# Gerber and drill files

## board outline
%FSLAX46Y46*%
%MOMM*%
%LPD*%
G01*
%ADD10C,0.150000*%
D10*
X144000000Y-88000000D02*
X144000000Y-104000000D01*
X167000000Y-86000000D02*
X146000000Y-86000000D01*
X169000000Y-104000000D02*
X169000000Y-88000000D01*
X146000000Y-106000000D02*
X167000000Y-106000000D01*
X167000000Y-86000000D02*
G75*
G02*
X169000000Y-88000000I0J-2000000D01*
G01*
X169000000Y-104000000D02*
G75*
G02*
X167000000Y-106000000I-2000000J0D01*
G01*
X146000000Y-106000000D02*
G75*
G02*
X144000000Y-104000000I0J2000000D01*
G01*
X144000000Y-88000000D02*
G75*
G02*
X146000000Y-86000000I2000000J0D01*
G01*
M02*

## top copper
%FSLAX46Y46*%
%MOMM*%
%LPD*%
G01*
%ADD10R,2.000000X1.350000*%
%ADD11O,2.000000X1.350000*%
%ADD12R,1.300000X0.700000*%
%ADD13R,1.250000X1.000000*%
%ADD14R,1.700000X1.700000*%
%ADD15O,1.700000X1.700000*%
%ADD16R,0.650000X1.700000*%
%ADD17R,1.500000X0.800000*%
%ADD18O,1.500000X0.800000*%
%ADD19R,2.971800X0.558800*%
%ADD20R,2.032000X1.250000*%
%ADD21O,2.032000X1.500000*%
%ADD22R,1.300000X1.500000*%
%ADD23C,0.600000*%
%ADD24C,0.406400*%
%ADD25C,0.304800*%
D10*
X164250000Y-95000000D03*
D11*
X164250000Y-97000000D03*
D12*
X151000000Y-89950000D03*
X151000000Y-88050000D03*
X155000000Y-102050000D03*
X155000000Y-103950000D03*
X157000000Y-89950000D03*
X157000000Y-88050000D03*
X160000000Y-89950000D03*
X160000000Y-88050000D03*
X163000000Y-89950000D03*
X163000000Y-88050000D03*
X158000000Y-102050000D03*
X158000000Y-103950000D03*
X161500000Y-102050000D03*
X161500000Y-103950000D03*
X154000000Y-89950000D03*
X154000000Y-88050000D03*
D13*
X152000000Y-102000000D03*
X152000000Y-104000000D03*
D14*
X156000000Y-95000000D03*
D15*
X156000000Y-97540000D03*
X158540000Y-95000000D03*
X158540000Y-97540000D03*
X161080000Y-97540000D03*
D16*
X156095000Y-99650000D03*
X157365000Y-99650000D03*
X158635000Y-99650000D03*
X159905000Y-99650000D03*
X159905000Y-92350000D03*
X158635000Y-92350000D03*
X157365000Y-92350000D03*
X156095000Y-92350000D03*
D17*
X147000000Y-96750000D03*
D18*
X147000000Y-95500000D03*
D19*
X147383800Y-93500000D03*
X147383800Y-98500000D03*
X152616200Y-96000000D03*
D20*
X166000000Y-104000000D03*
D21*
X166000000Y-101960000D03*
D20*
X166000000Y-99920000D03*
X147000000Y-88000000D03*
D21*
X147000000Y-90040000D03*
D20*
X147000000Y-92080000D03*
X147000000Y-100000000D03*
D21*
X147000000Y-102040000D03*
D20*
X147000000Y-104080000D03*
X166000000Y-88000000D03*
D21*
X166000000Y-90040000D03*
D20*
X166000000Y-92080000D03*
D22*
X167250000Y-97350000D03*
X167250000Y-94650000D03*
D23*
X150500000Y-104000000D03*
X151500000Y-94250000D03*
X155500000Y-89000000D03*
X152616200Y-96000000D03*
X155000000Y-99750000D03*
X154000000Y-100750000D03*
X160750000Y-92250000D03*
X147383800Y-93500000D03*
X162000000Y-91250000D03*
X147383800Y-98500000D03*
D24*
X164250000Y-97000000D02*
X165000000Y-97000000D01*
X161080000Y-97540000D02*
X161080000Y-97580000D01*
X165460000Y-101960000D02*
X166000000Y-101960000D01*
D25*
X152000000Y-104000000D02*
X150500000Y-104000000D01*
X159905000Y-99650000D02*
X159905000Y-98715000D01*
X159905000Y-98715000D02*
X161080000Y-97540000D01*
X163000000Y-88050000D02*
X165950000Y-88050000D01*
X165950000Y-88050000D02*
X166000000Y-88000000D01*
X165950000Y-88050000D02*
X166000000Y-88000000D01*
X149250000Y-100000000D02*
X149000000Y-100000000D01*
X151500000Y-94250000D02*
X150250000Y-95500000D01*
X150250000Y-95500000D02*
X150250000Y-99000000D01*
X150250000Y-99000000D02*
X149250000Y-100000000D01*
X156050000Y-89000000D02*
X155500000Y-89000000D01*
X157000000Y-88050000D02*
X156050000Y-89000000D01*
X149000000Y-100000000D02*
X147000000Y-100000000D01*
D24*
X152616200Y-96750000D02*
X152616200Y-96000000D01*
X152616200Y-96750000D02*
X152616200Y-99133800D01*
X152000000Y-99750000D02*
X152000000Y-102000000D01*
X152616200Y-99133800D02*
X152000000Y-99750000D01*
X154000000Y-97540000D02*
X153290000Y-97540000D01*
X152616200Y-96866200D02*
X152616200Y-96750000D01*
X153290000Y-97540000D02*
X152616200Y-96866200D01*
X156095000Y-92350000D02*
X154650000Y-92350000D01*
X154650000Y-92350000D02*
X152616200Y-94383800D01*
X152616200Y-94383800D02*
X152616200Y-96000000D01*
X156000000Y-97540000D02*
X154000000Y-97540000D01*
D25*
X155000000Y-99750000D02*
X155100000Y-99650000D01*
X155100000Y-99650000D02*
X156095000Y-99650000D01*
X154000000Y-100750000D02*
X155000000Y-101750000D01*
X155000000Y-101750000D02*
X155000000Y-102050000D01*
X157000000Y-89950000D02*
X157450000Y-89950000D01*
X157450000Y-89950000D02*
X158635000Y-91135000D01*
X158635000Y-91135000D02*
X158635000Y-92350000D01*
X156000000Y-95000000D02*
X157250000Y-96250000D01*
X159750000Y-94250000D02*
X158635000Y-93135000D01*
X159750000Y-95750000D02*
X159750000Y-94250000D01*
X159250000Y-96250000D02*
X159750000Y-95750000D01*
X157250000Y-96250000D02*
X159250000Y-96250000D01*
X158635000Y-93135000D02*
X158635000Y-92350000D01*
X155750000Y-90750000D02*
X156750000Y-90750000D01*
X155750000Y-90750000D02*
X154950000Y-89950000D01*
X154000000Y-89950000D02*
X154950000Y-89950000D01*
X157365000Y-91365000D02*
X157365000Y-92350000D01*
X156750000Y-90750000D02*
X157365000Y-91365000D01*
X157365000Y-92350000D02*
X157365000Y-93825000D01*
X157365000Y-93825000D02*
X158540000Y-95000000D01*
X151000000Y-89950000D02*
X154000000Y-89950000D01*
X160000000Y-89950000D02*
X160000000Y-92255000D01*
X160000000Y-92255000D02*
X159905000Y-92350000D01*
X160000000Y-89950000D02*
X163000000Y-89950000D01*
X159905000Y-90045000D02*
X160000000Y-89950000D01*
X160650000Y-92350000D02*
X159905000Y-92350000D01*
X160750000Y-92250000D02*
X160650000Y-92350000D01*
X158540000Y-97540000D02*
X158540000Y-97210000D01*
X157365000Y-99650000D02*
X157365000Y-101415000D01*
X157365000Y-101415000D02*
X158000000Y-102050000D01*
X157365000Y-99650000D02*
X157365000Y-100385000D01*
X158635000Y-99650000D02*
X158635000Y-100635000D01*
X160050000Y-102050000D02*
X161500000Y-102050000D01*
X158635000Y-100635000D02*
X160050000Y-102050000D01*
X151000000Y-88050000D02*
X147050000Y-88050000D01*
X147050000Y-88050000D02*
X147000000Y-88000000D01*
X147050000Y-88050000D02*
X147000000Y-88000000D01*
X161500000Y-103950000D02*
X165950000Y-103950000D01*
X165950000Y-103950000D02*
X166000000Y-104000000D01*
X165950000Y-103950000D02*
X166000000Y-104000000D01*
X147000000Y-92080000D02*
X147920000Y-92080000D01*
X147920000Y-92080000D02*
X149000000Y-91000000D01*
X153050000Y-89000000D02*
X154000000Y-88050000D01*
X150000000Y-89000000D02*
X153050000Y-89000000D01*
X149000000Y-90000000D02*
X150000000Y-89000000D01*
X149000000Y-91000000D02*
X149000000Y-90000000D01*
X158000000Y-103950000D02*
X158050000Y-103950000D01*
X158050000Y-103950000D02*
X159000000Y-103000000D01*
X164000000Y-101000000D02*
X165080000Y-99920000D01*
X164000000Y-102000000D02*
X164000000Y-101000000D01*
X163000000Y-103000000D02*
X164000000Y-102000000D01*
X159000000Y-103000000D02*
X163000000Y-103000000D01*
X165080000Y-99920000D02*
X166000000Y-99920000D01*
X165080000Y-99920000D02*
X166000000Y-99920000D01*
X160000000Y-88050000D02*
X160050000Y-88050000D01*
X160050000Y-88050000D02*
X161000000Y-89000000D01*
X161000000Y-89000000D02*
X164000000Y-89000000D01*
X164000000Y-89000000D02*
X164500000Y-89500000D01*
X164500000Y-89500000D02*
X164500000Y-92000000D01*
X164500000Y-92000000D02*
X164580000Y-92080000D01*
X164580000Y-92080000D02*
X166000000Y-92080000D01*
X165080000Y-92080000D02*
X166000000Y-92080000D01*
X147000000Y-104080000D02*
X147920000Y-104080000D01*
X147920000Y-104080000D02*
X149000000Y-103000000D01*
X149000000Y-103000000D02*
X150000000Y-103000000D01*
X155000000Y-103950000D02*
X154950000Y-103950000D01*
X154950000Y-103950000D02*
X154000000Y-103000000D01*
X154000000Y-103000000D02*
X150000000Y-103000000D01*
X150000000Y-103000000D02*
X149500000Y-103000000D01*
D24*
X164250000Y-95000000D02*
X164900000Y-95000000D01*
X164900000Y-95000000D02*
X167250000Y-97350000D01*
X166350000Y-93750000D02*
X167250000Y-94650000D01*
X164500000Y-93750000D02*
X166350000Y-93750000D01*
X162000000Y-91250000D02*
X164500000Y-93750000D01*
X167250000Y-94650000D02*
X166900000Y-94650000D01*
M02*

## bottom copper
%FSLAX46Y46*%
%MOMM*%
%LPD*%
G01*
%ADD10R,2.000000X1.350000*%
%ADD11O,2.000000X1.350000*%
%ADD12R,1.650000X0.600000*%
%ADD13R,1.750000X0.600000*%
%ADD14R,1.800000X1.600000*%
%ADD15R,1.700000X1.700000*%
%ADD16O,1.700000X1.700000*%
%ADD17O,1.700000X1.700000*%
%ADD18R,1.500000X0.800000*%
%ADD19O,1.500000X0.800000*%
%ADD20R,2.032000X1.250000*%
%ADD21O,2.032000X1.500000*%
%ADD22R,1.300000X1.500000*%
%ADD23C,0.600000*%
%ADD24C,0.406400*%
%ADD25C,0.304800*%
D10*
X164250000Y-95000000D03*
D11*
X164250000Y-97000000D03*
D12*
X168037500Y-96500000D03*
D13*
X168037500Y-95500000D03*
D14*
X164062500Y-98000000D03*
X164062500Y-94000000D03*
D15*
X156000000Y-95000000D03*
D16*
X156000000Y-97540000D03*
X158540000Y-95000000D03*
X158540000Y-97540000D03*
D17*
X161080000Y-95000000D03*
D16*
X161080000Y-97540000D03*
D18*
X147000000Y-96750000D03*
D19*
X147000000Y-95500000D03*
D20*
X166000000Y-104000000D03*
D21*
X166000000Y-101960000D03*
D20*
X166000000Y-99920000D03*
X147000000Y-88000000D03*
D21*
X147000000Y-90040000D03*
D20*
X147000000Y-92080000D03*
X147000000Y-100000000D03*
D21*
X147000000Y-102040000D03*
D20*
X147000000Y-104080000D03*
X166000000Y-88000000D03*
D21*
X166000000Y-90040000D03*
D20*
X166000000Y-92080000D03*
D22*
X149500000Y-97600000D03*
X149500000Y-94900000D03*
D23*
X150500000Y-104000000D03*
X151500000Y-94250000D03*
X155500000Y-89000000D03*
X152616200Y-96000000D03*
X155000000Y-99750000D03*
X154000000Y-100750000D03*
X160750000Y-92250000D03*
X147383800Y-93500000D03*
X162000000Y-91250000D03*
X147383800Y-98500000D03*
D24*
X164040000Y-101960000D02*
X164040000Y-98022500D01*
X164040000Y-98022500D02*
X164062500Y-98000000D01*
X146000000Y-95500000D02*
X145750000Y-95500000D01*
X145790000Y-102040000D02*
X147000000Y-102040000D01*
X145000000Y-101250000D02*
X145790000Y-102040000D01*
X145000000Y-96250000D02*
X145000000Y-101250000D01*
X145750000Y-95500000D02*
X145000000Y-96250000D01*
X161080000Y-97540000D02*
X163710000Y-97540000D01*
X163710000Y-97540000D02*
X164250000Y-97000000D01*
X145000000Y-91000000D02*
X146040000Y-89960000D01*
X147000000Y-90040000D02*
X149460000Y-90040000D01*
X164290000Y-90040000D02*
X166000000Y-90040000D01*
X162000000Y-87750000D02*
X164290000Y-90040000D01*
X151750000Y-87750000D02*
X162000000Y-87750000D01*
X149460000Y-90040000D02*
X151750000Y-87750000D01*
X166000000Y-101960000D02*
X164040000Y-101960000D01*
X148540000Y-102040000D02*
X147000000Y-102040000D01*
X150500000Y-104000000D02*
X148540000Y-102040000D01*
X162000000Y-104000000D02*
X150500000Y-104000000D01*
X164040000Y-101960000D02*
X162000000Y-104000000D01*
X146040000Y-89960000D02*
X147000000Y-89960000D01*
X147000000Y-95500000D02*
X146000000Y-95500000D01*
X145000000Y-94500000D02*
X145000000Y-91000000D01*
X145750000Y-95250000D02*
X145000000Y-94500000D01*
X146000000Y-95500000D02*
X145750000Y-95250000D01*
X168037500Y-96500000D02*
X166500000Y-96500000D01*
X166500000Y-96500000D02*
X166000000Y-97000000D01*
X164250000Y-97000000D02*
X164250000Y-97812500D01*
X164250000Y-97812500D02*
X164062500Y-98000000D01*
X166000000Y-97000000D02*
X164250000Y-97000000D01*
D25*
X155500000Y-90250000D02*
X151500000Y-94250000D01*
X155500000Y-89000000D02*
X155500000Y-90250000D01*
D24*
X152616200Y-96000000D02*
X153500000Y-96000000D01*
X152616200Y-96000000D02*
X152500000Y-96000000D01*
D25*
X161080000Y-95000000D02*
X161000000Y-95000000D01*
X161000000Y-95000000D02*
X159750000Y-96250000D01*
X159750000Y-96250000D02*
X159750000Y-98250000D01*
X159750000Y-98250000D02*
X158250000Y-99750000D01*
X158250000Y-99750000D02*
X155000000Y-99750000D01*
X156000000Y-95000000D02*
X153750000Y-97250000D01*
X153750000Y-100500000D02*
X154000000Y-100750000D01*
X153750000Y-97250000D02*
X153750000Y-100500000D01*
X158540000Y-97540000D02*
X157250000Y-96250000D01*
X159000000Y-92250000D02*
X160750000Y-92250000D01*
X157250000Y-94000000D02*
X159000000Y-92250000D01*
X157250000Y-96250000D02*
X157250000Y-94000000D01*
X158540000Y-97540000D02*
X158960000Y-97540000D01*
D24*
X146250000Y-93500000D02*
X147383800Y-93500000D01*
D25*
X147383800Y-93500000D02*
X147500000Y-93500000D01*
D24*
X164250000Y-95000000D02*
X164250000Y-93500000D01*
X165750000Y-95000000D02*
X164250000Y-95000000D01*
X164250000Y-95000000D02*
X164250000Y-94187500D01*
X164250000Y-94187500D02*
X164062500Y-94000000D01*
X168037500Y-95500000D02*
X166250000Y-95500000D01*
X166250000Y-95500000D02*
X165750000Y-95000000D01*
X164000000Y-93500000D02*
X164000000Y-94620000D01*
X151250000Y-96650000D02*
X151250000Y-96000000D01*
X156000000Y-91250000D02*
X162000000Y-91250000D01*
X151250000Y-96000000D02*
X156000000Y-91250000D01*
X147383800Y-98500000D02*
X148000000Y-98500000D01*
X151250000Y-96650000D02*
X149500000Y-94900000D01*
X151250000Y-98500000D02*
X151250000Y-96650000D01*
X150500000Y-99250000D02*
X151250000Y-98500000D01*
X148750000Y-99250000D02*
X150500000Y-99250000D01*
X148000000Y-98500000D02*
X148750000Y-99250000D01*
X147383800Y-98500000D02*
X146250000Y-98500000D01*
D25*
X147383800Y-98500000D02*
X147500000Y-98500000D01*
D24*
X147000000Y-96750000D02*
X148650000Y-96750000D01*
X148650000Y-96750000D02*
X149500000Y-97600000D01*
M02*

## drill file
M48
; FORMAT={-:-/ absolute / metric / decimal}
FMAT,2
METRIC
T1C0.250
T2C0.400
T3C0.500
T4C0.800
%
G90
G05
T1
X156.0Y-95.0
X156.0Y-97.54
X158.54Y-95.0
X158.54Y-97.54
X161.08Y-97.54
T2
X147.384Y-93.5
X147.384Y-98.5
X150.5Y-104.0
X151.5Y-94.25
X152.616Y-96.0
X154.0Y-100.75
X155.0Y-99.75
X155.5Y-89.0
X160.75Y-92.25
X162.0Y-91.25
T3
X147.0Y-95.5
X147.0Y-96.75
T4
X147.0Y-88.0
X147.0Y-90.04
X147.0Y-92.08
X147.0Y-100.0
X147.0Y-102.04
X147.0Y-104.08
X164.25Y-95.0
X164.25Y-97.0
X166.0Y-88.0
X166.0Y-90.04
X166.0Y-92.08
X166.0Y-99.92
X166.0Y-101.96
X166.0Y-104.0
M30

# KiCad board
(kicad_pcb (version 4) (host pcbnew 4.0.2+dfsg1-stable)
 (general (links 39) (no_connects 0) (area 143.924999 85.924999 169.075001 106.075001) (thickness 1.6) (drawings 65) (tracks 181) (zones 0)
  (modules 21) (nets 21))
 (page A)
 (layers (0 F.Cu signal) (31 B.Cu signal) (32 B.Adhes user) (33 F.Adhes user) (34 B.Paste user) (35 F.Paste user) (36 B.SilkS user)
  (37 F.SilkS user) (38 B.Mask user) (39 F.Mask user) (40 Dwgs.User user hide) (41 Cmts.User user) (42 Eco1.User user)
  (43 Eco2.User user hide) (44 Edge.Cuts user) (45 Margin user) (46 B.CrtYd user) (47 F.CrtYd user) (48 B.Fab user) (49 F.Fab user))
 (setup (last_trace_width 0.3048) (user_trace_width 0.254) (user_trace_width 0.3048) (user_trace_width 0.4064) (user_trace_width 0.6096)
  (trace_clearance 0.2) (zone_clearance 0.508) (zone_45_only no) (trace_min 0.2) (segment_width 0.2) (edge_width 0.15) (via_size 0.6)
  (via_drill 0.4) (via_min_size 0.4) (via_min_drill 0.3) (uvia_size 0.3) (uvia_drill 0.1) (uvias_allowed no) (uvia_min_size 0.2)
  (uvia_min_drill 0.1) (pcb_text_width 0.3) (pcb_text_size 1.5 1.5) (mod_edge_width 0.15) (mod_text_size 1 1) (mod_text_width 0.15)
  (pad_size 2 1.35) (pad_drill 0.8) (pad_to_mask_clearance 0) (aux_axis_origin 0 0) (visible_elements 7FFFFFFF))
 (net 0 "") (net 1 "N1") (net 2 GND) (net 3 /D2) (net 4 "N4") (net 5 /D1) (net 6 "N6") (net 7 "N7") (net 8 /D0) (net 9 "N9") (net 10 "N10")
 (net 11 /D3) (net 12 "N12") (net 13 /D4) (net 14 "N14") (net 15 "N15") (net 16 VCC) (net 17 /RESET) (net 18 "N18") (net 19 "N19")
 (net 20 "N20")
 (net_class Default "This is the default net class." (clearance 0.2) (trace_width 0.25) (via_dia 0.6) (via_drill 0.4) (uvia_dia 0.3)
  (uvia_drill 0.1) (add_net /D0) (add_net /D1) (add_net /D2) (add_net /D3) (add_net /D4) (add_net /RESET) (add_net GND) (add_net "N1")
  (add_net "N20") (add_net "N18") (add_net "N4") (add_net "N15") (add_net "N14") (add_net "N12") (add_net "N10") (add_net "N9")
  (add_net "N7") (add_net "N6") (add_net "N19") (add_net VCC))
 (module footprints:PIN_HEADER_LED (layer B.Cu) (at 164.25 95 180)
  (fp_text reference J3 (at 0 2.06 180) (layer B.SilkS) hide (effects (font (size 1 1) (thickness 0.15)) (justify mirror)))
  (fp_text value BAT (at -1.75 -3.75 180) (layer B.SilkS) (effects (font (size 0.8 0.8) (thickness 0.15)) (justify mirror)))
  (pad 1 thru_hole rect (at 0 0 180) (size 2 1.35) (drill 0.8) (layers *.Cu *.Mask) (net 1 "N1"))
  (pad 2 thru_hole oval (at 0 -2 180) (size 2 1.35) (drill 0.8) (layers *.Cu *.Mask) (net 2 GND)))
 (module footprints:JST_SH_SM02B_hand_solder (layer B.Cu) (at 166 96 90)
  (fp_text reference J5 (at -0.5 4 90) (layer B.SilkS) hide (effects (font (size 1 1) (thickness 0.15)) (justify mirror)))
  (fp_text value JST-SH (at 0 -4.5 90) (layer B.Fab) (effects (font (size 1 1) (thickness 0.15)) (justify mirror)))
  (pad 1 smd rect (at -0.5 2.0375 90) (size 0.6 1.65) (layers B.Cu B.Paste B.Mask) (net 2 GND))
  (pad 2 smd rect (at 0.5 2.0375 90) (size 0.6 1.75) (layers B.Cu B.Paste B.Mask) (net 1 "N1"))
  (pad 1 smd rect (at -2 -1.9375 90) (size 1.6 1.8) (layers B.Cu B.Paste B.Mask) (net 2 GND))
  (pad 2 smd rect (at 2 -1.9375 90) (size 1.6 1.8) (layers B.Cu B.Paste B.Mask) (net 1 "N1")))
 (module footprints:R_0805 (layer F.Cu) (at 151 89 90)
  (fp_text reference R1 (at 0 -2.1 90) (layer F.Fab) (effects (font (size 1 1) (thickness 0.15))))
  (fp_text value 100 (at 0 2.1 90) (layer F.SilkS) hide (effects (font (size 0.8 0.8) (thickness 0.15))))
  (pad 1 smd rect (at -0.95 0 90) (size 0.7 1.3) (layers F.Cu F.Paste F.Mask) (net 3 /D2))
  (pad 2 smd rect (at 0.95 0 90) (size 0.7 1.3) (layers F.Cu F.Paste F.Mask) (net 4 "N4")))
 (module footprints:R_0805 (layer F.Cu) (at 155 103 270)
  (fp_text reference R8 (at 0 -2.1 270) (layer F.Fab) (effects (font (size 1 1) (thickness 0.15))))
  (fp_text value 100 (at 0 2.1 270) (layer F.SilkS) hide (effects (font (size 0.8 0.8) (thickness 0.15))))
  (pad 1 smd rect (at -0.95 0 270) (size 0.7 1.3) (layers F.Cu F.Paste F.Mask) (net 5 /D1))
  (pad 2 smd rect (at 0.95 0 270) (size 0.7 1.3) (layers F.Cu F.Paste F.Mask) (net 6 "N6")))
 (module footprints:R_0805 (layer F.Cu) (at 157 89 90)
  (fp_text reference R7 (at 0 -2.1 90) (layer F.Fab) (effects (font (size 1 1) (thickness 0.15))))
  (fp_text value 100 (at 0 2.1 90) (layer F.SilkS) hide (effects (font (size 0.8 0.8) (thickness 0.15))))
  (pad 1 smd rect (at -0.95 0 90) (size 0.7 1.3) (layers F.Cu F.Paste F.Mask) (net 5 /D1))
  (pad 2 smd rect (at 0.95 0 90) (size 0.7 1.3) (layers F.Cu F.Paste F.Mask) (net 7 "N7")))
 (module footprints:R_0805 (layer F.Cu) (at 160 89 90)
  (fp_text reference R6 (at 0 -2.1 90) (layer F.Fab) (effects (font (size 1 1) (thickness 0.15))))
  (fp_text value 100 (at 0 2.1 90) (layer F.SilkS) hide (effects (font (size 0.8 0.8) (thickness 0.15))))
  (pad 1 smd rect (at -0.95 0 90) (size 0.7 1.3) (layers F.Cu F.Paste F.Mask) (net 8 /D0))
  (pad 2 smd rect (at 0.95 0 90) (size 0.7 1.3) (layers F.Cu F.Paste F.Mask) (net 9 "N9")))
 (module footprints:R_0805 (layer F.Cu) (at 163 89 90)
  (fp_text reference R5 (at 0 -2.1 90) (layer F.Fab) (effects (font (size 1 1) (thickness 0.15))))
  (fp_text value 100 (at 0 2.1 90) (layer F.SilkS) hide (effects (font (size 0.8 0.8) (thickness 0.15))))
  (pad 1 smd rect (at -0.95 0 90) (size 0.7 1.3) (layers F.Cu F.Paste F.Mask) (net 8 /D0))
  (pad 2 smd rect (at 0.95 0 90) (size 0.7 1.3) (layers F.Cu F.Paste F.Mask) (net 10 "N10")))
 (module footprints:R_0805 (layer F.Cu) (at 158 103 270)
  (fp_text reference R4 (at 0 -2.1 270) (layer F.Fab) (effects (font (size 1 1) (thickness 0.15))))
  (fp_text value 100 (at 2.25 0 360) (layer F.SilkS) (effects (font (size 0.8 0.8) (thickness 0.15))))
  (pad 1 smd rect (at -0.95 0 270) (size 0.7 1.3) (layers F.Cu F.Paste F.Mask) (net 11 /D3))
  (pad 2 smd rect (at 0.95 0 270) (size 0.7 1.3) (layers F.Cu F.Paste F.Mask) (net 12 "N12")))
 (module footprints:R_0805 (layer F.Cu) (at 161.5 103 270)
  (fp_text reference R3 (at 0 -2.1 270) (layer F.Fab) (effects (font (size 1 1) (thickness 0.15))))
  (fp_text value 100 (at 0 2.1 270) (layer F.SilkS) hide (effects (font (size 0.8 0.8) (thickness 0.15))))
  (pad 1 smd rect (at -0.95 0 270) (size 0.7 1.3) (layers F.Cu F.Paste F.Mask) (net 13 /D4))
  (pad 2 smd rect (at 0.95 0 270) (size 0.7 1.3) (layers F.Cu F.Paste F.Mask) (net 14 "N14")))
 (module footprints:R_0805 (layer F.Cu) (at 154 89 90)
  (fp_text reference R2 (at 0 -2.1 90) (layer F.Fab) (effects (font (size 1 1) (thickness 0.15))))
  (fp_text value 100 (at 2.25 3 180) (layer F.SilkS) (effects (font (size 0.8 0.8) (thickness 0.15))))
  (pad 1 smd rect (at -0.95 0 90) (size 0.7 1.3) (layers F.Cu F.Paste F.Mask) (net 3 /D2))
  (pad 2 smd rect (at 0.95 0 90) (size 0.7 1.3) (layers F.Cu F.Paste F.Mask) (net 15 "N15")))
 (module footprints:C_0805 (layer F.Cu) (at 152 103 270)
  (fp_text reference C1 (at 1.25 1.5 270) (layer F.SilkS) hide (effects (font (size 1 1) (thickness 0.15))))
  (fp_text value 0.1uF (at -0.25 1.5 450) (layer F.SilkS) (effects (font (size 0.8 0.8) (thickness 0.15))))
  (pad 1 smd rect (at -1 0 270) (size 1 1.25) (layers F.Cu F.Paste F.Mask) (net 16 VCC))
  (pad 2 smd rect (at 1 0 270) (size 1 1.25) (layers F.Cu F.Paste F.Mask) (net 2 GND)))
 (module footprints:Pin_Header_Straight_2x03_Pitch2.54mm (layer B.Cu) (at 156 95 270)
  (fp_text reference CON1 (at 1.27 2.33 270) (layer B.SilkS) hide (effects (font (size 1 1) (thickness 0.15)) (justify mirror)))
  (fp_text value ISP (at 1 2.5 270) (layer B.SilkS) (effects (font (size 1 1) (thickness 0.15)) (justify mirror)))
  (pad 1 thru_hole rect (at 0 0 270) (size 1.7 1.7) (drill 0.25) (layers *.Cu B.SilkS B.Mask) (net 5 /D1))
  (pad 2 thru_hole oval (at 2.54 0 270) (size 1.7 1.7) (drill 0.25) (layers *.Cu B.SilkS B.Mask) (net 16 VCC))
  (pad 3 thru_hole oval (at 0 -2.54 270) (size 1.7 1.7) (drill 0.25) (layers *.Cu B.SilkS B.Mask) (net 3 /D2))
  (pad 4 thru_hole oval (at 2.54 -2.54 270) (size 1.7 1.7) (drill 0.25) (layers *.Cu B.SilkS B.Mask) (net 8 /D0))
  (pad 5 smd oval (at 0 -5.08 270) (size 1.7 1.7) (layers B.Cu B.Paste B.Mask) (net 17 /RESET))
  (pad 6 thru_hole oval (at 2.54 -5.08 270) (size 1.7 1.7) (drill 0.25) (layers *.Cu B.SilkS B.Mask) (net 2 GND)))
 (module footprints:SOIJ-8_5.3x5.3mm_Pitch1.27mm (layer F.Cu) (at 158 96 90)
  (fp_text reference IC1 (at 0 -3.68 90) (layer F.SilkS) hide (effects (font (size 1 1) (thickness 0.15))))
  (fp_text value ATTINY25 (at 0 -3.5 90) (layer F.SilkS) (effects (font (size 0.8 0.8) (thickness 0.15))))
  (pad 1 smd rect (at -3.65 -1.905 90) (size 1.7 0.65) (layers F.Cu F.Paste F.Mask) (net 17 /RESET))
  (pad 2 smd rect (at -3.65 -0.635 90) (size 1.7 0.65) (layers F.Cu F.Paste F.Mask) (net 11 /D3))
  (pad 3 smd rect (at -3.65 0.635 90) (size 1.7 0.65) (layers F.Cu F.Paste F.Mask) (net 13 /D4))
  (pad 4 smd rect (at -3.65 1.905 90) (size 1.7 0.65) (layers F.Cu F.Paste F.Mask) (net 2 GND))
  (pad 5 smd rect (at 3.65 1.905 90) (size 1.7 0.65) (layers F.Cu F.Paste F.Mask) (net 8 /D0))
  (pad 6 smd rect (at 3.65 0.635 90) (size 1.7 0.65) (layers F.Cu F.Paste F.Mask) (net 5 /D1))
  (pad 7 smd rect (at 3.65 -0.635 90) (size 1.7 0.65) (layers F.Cu F.Paste F.Mask) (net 3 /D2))
  (pad 8 smd rect (at 3.65 -1.905 90) (size 1.7 0.65) (layers F.Cu F.Paste F.Mask) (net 16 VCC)))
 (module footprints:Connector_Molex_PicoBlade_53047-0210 (layer F.Cu) (at 147 96.75 90)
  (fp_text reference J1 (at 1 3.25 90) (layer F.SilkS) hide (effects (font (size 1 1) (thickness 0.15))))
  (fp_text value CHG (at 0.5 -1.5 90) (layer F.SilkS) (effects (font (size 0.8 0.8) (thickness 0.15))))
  (pad 1 thru_hole rect (at 0 0 90) (size 0.8 1.5) (drill 0.5) (layers *.Cu *.Mask F.SilkS) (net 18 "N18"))
  (pad 2 thru_hole oval (at 1.25 0 90) (size 0.8 1.5) (drill 0.5) (layers *.Cu *.Mask F.SilkS) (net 2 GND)))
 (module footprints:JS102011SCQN (layer F.Cu) (at 150 96)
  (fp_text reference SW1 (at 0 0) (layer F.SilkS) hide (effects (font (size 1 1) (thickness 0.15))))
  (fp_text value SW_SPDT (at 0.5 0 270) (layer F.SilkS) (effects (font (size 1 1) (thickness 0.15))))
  (pad 1 smd rect (at -2.6162 -2.5) (size 2.9718 0.5588) (layers F.Cu F.Paste F.Mask) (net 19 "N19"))
  (pad 3 smd rect (at -2.6162 2.5) (size 2.9718 0.5588) (layers F.Cu F.Paste F.Mask) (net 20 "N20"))
  (pad 2 smd rect (at 2.6162 0) (size 2.9718 0.5588) (layers F.Cu F.Paste F.Mask) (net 16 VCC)))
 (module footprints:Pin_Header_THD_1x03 (layer F.Cu) (at 166 104 180)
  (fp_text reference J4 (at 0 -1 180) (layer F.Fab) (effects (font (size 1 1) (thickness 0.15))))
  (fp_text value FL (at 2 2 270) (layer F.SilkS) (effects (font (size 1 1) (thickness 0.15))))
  (pad 1 thru_hole rect (at 0 0 180) (size 2.032 1.25) (drill 0.8) (layers *.Cu *.Mask F.SilkS) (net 14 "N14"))
  (pad 2 thru_hole oval (at 0 2.04 180) (size 2.032 1.5) (drill 0.8) (layers *.Cu *.Mask F.SilkS) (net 2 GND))
  (pad 3 thru_hole rect (at 0 4.08 180) (size 2.032 1.25) (drill 0.8) (layers *.Cu *.Mask F.SilkS) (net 12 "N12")))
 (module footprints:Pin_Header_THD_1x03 (layer F.Cu) (at 147 88)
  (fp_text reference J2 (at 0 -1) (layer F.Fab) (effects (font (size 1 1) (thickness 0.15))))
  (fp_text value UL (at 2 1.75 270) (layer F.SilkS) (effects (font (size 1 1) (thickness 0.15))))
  (pad 1 thru_hole rect (at 0 0) (size 2.032 1.25) (drill 0.8) (layers *.Cu *.Mask F.SilkS) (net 4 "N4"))
  (pad 2 thru_hole oval (at 0 2.04) (size 2.032 1.5) (drill 0.8) (layers *.Cu *.Mask F.SilkS) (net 2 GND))
  (pad 3 thru_hole rect (at 0 4.08) (size 2.032 1.25) (drill 0.8) (layers *.Cu *.Mask F.SilkS) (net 15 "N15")))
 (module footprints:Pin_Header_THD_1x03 (layer F.Cu) (at 147 100)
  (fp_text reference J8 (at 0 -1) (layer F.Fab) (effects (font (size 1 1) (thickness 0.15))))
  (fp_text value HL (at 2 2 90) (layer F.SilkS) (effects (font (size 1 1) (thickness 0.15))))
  (pad 1 thru_hole rect (at 0 0) (size 2.032 1.25) (drill 0.8) (layers *.Cu *.Mask F.SilkS) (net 7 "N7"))
  (pad 2 thru_hole oval (at 0 2.04) (size 2.032 1.5) (drill 0.8) (layers *.Cu *.Mask F.SilkS) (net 2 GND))
  (pad 3 thru_hole rect (at 0 4.08) (size 2.032 1.25) (drill 0.8) (layers *.Cu *.Mask F.SilkS) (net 6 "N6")))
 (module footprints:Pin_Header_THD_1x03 (layer F.Cu) (at 166 88)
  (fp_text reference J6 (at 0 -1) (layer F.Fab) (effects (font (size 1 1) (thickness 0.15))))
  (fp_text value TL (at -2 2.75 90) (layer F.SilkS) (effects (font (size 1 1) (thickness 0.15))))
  (pad 1 thru_hole rect (at 0 0) (size 2.032 1.25) (drill 0.8) (layers *.Cu *.Mask F.SilkS) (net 10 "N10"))
  (pad 2 thru_hole oval (at 0 2.04) (size 2.032 1.5) (drill 0.8) (layers *.Cu *.Mask F.SilkS) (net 2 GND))
  (pad 3 thru_hole rect (at 0 4.08) (size 2.032 1.25) (drill 0.8) (layers *.Cu *.Mask F.SilkS) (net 9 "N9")))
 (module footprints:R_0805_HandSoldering (layer F.Cu) (at 167.25 96 90)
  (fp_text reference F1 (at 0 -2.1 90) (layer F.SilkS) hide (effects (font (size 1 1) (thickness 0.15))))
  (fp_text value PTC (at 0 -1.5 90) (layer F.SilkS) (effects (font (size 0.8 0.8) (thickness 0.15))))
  (pad 1 smd rect (at -1.35 0 90) (size 1.5 1.3) (layers F.Cu F.Paste F.Mask) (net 1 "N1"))
  (pad 2 smd rect (at 1.35 0 90) (size 1.5 1.3) (layers F.Cu F.Paste F.Mask) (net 20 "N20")))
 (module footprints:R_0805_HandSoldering (layer B.Cu) (at 149.5 96.25 90)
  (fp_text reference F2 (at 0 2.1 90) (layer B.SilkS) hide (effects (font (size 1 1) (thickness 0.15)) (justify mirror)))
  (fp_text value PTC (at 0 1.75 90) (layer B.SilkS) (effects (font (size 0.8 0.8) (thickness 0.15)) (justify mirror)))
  (pad 1 smd rect (at -1.35 0 90) (size 1.5 1.3) (layers B.Cu B.Paste B.Mask) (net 18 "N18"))
  (pad 2 smd rect (at 1.35 0 90) (size 1.5 1.3) (layers B.Cu B.Paste B.Mask) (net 20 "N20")))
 (gr_line (start 144 88) (end 144 104) (angle 90) (layer Edge.Cuts) (width 0.15))
 (gr_line (start 167 86) (end 146 86) (angle 90) (layer Edge.Cuts) (width 0.15))
 (gr_line (start 169 104) (end 169 88) (angle 90) (layer Edge.Cuts) (width 0.15))
 (gr_line (start 146 106) (end 167 106) (angle 90) (layer Edge.Cuts) (width 0.15))
 (gr_arc (start 167 88) (end 167 86) (angle 90) (layer Edge.Cuts) (width 0.15))
 (gr_arc (start 167 104) (end 169 104) (angle 90) (layer Edge.Cuts) (width 0.15))
 (gr_arc (start 146 104) (end 146 106) (angle 90) (layer Edge.Cuts) (width 0.15))
 (gr_arc (start 146 88) (end 144 88) (angle 90) (layer Edge.Cuts) (width 0.15))
 (segment (start 164.04 101.96) (end 164.04 98.0225) (width 0.4064) (layer B.Cu) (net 2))
 (segment (start 164.04 98.0225) (end 164.0625 98) (width 0.4064) (layer B.Cu) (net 2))
 (segment (start 146 95.5) (end 145.75 95.5) (width 0.4064) (layer B.Cu) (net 2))
 (segment (start 145.79 102.04) (end 147 102.04) (width 0.4064) (layer B.Cu) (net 2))
 (segment (start 145 101.25) (end 145.79 102.04) (width 0.4064) (layer B.Cu) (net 2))
 (segment (start 145 96.25) (end 145 101.25) (width 0.4064) (layer B.Cu) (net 2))
 (segment (start 145.75 95.5) (end 145 96.25) (width 0.4064) (layer B.Cu) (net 2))
 (segment (start 164.25 97) (end 165 97) (width 0.4064) (layer F.Cu) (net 2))
 (segment (start 161.08 97.54) (end 163.71 97.54) (width 0.4064) (layer B.Cu) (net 2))
 (segment (start 163.71 97.54) (end 164.25 97) (width 0.4064) (layer B.Cu) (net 2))
 (segment (start 145 91) (end 146.04 89.96) (width 0.4064) (layer B.Cu) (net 2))
 (segment (start 161.08 97.54) (end 161.08 97.58) (width 0.4064) (layer F.Cu) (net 2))
 (segment (start 165.46 101.96) (end 166 101.96) (width 0.4064) (layer F.Cu) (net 2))
 (segment (start 147 90.04) (end 149.46 90.04) (width 0.4064) (layer B.Cu) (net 2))
 (segment (start 164.29 90.04) (end 166 90.04) (width 0.4064) (layer B.Cu) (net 2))
 (segment (start 162 87.75) (end 164.29 90.04) (width 0.4064) (layer B.Cu) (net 2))
 (segment (start 151.75 87.75) (end 162 87.75) (width 0.4064) (layer B.Cu) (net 2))
 (segment (start 149.46 90.04) (end 151.75 87.75) (width 0.4064) (layer B.Cu) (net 2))
 (segment (start 152 104) (end 150.5 104) (width 0.3048) (layer F.Cu) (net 2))
 (via (at 150.5 104) (size 0.6) (drill 0.4) (layers F.Cu B.Cu) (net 2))
 (segment (start 166 101.96) (end 164.04 101.96) (width 0.4064) (layer B.Cu) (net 2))
 (segment (start 148.54 102.04) (end 147 102.04) (width 0.4064) (layer B.Cu) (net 2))
 (segment (start 150.5 104) (end 148.54 102.04) (width 0.4064) (layer B.Cu) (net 2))
 (segment (start 162 104) (end 150.5 104) (width 0.4064) (layer B.Cu) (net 2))
 (segment (start 164.04 101.96) (end 162 104) (width 0.4064) (layer B.Cu) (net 2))
 (segment (start 146.04 89.96) (end 147 89.96) (width 0.4064) (layer B.Cu) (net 2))
 (segment (start 159.905 99.65) (end 159.905 98.715) (width 0.3048) (layer F.Cu) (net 2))
 (segment (start 159.905 98.715) (end 161.08 97.54) (width 0.3048) (layer F.Cu) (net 2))
 (segment (start 147 95.5) (end 146 95.5) (width 0.4064) (layer B.Cu) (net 2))
 (segment (start 145 94.5) (end 145 91) (width 0.4064) (layer B.Cu) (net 2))
 (segment (start 145.75 95.25) (end 145 94.5) (width 0.4064) (layer B.Cu) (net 2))
 (segment (start 146 95.5) (end 145.75 95.25) (width 0.4064) (layer B.Cu) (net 2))
 (segment (start 168.0375 96.5) (end 166.5 96.5) (width 0.4064) (layer B.Cu) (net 2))
 (segment (start 166.5 96.5) (end 166 97) (width 0.4064) (layer B.Cu) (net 2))
 (segment (start 164.25 97) (end 164.25 97.8125) (width 0.4064) (layer B.Cu) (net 2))
 (segment (start 164.25 97.8125) (end 164.0625 98) (width 0.4064) (layer B.Cu) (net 2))
 (segment (start 166 97) (end 164.25 97) (width 0.4064) (layer B.Cu) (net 2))
 (segment (start 163 88.05) (end 165.95 88.05) (width 0.3048) (layer F.Cu) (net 10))
 (segment (start 165.95 88.05) (end 166 88) (width 0.3048) (layer F.Cu) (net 10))
 (segment (start 165.95 88.05) (end 166 88) (width 0.3048) (layer F.Cu) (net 10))
 (segment (start 149.25 100) (end 149 100) (width 0.3048) (layer F.Cu) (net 7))
 (segment (start 155.5 90.25) (end 151.5 94.25) (width 0.3048) (layer B.Cu) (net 7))
 (via (at 151.5 94.25) (size 0.6) (drill 0.4) (layers F.Cu B.Cu) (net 7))
 (segment (start 151.5 94.25) (end 150.25 95.5) (width 0.3048) (layer F.Cu) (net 7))
 (segment (start 150.25 95.5) (end 150.25 99) (width 0.3048) (layer F.Cu) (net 7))
 (segment (start 150.25 99) (end 149.25 100) (width 0.3048) (layer F.Cu) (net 7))
 (via (at 155.5 89) (size 0.6) (drill 0.4) (layers F.Cu B.Cu) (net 7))
 (segment (start 156.05 89) (end 155.5 89) (width 0.3048) (layer F.Cu) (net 7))
 (segment (start 157 88.05) (end 156.05 89) (width 0.3048) (layer F.Cu) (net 7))
 (segment (start 155.5 89) (end 155.5 90.25) (width 0.3048) (layer B.Cu) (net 7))
 (segment (start 149 100) (end 147 100) (width 0.3048) (layer F.Cu) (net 7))
 (segment (start 152.6162 96) (end 153.5 96) (width 0.4064) (layer B.Cu) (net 16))
 (segment (start 152.6162 96.75) (end 152.6162 96) (width 0.4064) (layer F.Cu) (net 16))
 (via (at 152.6162 96) (size 0.6) (drill 0.4) (layers F.Cu B.Cu) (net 16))
 (segment (start 152.6162 96) (end 152.5 96) (width 0.4064) (layer B.Cu) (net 16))
 (segment (start 152.6162 96.75) (end 152.6162 99.1338) (width 0.4064) (layer F.Cu) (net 16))
 (segment (start 152 99.75) (end 152 102) (width 0.4064) (layer F.Cu) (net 16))
 (segment (start 152.6162 99.1338) (end 152 99.75) (width 0.4064) (layer F.Cu) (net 16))
 (segment (start 154 97.54) (end 153.29 97.54) (width 0.4064) (layer F.Cu) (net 16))
 (segment (start 152.6162 96.8662) (end 152.6162 96.75) (width 0.4064) (layer F.Cu) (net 16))
 (segment (start 153.29 97.54) (end 152.6162 96.8662) (width 0.4064) (layer F.Cu) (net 16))
 (segment (start 156.095 92.35) (end 154.65 92.35) (width 0.4064) (layer F.Cu) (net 16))
 (segment (start 154.65 92.35) (end 152.6162 94.3838) (width 0.4064) (layer F.Cu) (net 16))
 (segment (start 152.6162 94.3838) (end 152.6162 96) (width 0.4064) (layer F.Cu) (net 16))
 (segment (start 156 97.54) (end 154 97.54) (width 0.4064) (layer F.Cu) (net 16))
 (segment (start 161.08 95) (end 161 95) (width 0.3048) (layer B.Cu) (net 17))
 (segment (start 161 95) (end 159.75 96.25) (width 0.3048) (layer B.Cu) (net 17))
 (segment (start 159.75 96.25) (end 159.75 98.25) (width 0.3048) (layer B.Cu) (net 17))
 (segment (start 159.75 98.25) (end 158.25 99.75) (width 0.3048) (layer B.Cu) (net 17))
 (segment (start 158.25 99.75) (end 155 99.75) (width 0.3048) (layer B.Cu) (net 17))
 (via (at 155 99.75) (size 0.6) (drill 0.4) (layers F.Cu B.Cu) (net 17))
 (segment (start 155 99.75) (end 155.1 99.65) (width 0.3048) (layer F.Cu) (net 17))
 (segment (start 155.1 99.65) (end 156.095 99.65) (width 0.3048) (layer F.Cu) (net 17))
 (segment (start 156 95) (end 153.75 97.25) (width 0.3048) (layer B.Cu) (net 5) (status 400000))
 (segment (start 154 100.75) (end 155 101.75) (width 0.3048) (layer F.Cu) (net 5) (status 800000))
 (via (at 154 100.75) (size 0.6) (drill 0.4) (layers F.Cu B.Cu) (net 5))
 (segment (start 153.75 100.5) (end 154 100.75) (width 0.3048) (layer B.Cu) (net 5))
 (segment (start 153.75 97.25) (end 153.75 100.5) (width 0.3048) (layer B.Cu) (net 5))
 (segment (start 155 101.75) (end 155 102.05) (width 0.3048) (layer F.Cu) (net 5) (status C00000))
 (segment (start 157 89.95) (end 157.45 89.95) (width 0.3048) (layer F.Cu) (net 5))
 (segment (start 157.45 89.95) (end 158.635 91.135) (width 0.3048) (layer F.Cu) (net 5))
 (segment (start 158.635 91.135) (end 158.635 92.35) (width 0.3048) (layer F.Cu) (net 5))
 (segment (start 156 95) (end 157.25 96.25) (width 0.3048) (layer F.Cu) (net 5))
 (segment (start 159.75 94.25) (end 158.635 93.135) (width 0.3048) (layer F.Cu) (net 5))
 (segment (start 159.75 95.75) (end 159.75 94.25) (width 0.3048) (layer F.Cu) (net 5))
 (segment (start 159.25 96.25) (end 159.75 95.75) (width 0.3048) (layer F.Cu) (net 5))
 (segment (start 157.25 96.25) (end 159.25 96.25) (width 0.3048) (layer F.Cu) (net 5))
 (segment (start 158.635 93.135) (end 158.635 92.35) (width 0.3048) (layer F.Cu) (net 5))
 (segment (start 155.75 90.75) (end 156.75 90.75) (width 0.3048) (layer F.Cu) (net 3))
 (segment (start 155.75 90.75) (end 154.95 89.95) (width 0.3048) (layer F.Cu) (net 3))
 (segment (start 154 89.95) (end 154.95 89.95) (width 0.3048) (layer F.Cu) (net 3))
 (segment (start 157.365 91.365) (end 157.365 92.35) (width 0.3048) (layer F.Cu) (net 3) (status 800000))
 (segment (start 156.75 90.75) (end 157.365 91.365) (width 0.3048) (layer F.Cu) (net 3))
 (segment (start 157.365 92.35) (end 157.365 93.825) (width 0.3048) (layer F.Cu) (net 3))
 (segment (start 157.365 93.825) (end 158.54 95) (width 0.3048) (layer F.Cu) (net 3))
 (segment (start 151 89.95) (end 154 89.95) (width 0.3048) (layer F.Cu) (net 3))
 (segment (start 160 89.95) (end 160 92.255) (width 0.3048) (layer F.Cu) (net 8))
 (segment (start 160 92.255) (end 159.905 92.35) (width 0.3048) (layer F.Cu) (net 8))
 (segment (start 160 89.95) (end 163 89.95) (width 0.3048) (layer F.Cu) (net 8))
 (segment (start 159.905 90.045) (end 160 89.95) (width 0.3048) (layer F.Cu) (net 8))
 (segment (start 158.54 97.54) (end 157.25 96.25) (width 0.3048) (layer B.Cu) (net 8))
 (segment (start 159 92.25) (end 160.75 92.25) (width 0.3048) (layer B.Cu) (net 8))
 (segment (start 157.25 94) (end 159 92.25) (width 0.3048) (layer B.Cu) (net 8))
 (segment (start 157.25 96.25) (end 157.25 94) (width 0.3048) (layer B.Cu) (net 8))
 (segment (start 158.54 97.54) (end 158.96 97.54) (width 0.3048) (layer B.Cu) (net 8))
 (segment (start 160.65 92.35) (end 159.905 92.35) (width 0.3048) (layer F.Cu) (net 8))
 (via (at 160.75 92.25) (size 0.6) (drill 0.4) (layers F.Cu B.Cu) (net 8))
 (segment (start 160.75 92.25) (end 160.65 92.35) (width 0.3048) (layer F.Cu) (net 8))
 (segment (start 158.54 97.54) (end 158.54 97.21) (width 0.3048) (layer F.Cu) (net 8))
 (segment (start 157.365 99.65) (end 157.365 101.415) (width 0.3048) (layer F.Cu) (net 11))
 (segment (start 157.365 101.415) (end 158 102.05) (width 0.3048) (layer F.Cu) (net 11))
 (segment (start 157.365 99.65) (end 157.365 100.385) (width 0.3048) (layer F.Cu) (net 11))
 (segment (start 158.635 99.65) (end 158.635 100.635) (width 0.3048) (layer F.Cu) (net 13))
 (segment (start 160.05 102.05) (end 161.5 102.05) (width 0.3048) (layer F.Cu) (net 13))
 (segment (start 158.635 100.635) (end 160.05 102.05) (width 0.3048) (layer F.Cu) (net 13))
 (segment (start 151 88.05) (end 147.05 88.05) (width 0.3048) (layer F.Cu) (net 4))
 (segment (start 147.05 88.05) (end 147 88) (width 0.3048) (layer F.Cu) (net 4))
 (segment (start 147.05 88.05) (end 147 88) (width 0.3048) (layer F.Cu) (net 4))
 (segment (start 161.5 103.95) (end 165.95 103.95) (width 0.3048) (layer F.Cu) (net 14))
 (segment (start 165.95 103.95) (end 166 104) (width 0.3048) (layer F.Cu) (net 14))
 (segment (start 165.95 103.95) (end 166 104) (width 0.3048) (layer F.Cu) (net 14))
 (segment (start 147 92.08) (end 147.92 92.08) (width 0.3048) (layer F.Cu) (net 15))
 (segment (start 147.92 92.08) (end 149 91) (width 0.3048) (layer F.Cu) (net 15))
 (segment (start 153.05 89) (end 154 88.05) (width 0.3048) (layer F.Cu) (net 15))
 (segment (start 150 89) (end 153.05 89) (width 0.3048) (layer F.Cu) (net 15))
 (segment (start 149 90) (end 150 89) (width 0.3048) (layer F.Cu) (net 15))
 (segment (start 149 91) (end 149 90) (width 0.3048) (layer F.Cu) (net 15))
 (segment (start 158 103.95) (end 158.05 103.95) (width 0.3048) (layer F.Cu) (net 12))
 (segment (start 158.05 103.95) (end 159 103) (width 0.3048) (layer F.Cu) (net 12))
 (segment (start 164 101) (end 165.08 99.92) (width 0.3048) (layer F.Cu) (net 12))
 (segment (start 164 102) (end 164 101) (width 0.3048) (layer F.Cu) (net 12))
 (segment (start 163 103) (end 164 102) (width 0.3048) (layer F.Cu) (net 12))
 (segment (start 159 103) (end 163 103) (width 0.3048) (layer F.Cu) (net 12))
 (segment (start 165.08 99.92) (end 166 99.92) (width 0.3048) (layer F.Cu) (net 12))
 (segment (start 165.08 99.92) (end 166 99.92) (width 0.3048) (layer F.Cu) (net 12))
 (segment (start 160 88.05) (end 160.05 88.05) (width 0.3048) (layer F.Cu) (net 9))
 (segment (start 160.05 88.05) (end 161 89) (width 0.3048) (layer F.Cu) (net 9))
 (segment (start 161 89) (end 164 89) (width 0.3048) (layer F.Cu) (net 9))
 (segment (start 164 89) (end 164.5 89.5) (width 0.3048) (layer F.Cu) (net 9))
 (segment (start 164.5 89.5) (end 164.5 92) (width 0.3048) (layer F.Cu) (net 9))
 (segment (start 164.5 92) (end 164.58 92.08) (width 0.3048) (layer F.Cu) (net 9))
 (segment (start 164.58 92.08) (end 166 92.08) (width 0.3048) (layer F.Cu) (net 9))
 (segment (start 165.08 92.08) (end 166 92.08) (width 0.3048) (layer F.Cu) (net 9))
 (segment (start 147 104.08) (end 147.92 104.08) (width 0.3048) (layer F.Cu) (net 6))
 (segment (start 147.92 104.08) (end 149 103) (width 0.3048) (layer F.Cu) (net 6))
 (segment (start 149 103) (end 150 103) (width 0.3048) (layer F.Cu) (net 6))
 (segment (start 155 103.95) (end 154.95 103.95) (width 0.3048) (layer F.Cu) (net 6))
 (segment (start 154.95 103.95) (end 154 103) (width 0.3048) (layer F.Cu) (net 6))
 (segment (start 154 103) (end 150 103) (width 0.3048) (layer F.Cu) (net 6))
 (segment (start 150 103) (end 149.5 103) (width 0.3048) (layer F.Cu) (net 6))
 (segment (start 146.25 93.5) (end 147.3838 93.5) (width 0.4064) (layer B.Cu) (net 19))
 (segment (start 147.3838 93.5) (end 147.5 93.5) (width 0.3048) (layer B.Cu) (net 19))
 (via (at 147.3838 93.5) (size 0.6) (drill 0.4) (layers F.Cu B.Cu) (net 19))
 (segment (start 164.25 95) (end 164.9 95) (width 0.4064) (layer F.Cu) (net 1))
 (segment (start 164.9 95) (end 167.25 97.35) (width 0.4064) (layer F.Cu) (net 1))
 (segment (start 164.25 95) (end 164.25 93.5) (width 0.4064) (layer B.Cu) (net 1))
 (segment (start 165.75 95) (end 164.25 95) (width 0.4064) (layer B.Cu) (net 1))
 (segment (start 164.25 95) (end 164.25 94.1875) (width 0.4064) (layer B.Cu) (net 1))
 (segment (start 164.25 94.1875) (end 164.0625 94) (width 0.4064) (layer B.Cu) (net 1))
 (segment (start 168.0375 95.5) (end 166.25 95.5) (width 0.4064) (layer B.Cu) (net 1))
 (segment (start 166.25 95.5) (end 165.75 95) (width 0.4064) (layer B.Cu) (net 1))
 (segment (start 164 93.5) (end 164 94.62) (width 0.4064) (layer B.Cu) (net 1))
 (segment (start 151.25 96.65) (end 151.25 96) (width 0.4064) (layer B.Cu) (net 20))
 (segment (start 166.35 93.75) (end 167.25 94.65) (width 0.4064) (layer F.Cu) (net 20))
 (segment (start 164.5 93.75) (end 166.35 93.75) (width 0.4064) (layer F.Cu) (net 20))
 (segment (start 162 91.25) (end 164.5 93.75) (width 0.4064) (layer F.Cu) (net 20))
 (via (at 162 91.25) (size 0.6) (drill 0.4) (layers F.Cu B.Cu) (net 20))
 (segment (start 156 91.25) (end 162 91.25) (width 0.4064) (layer B.Cu) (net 20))
 (segment (start 151.25 96) (end 156 91.25) (width 0.4064) (layer B.Cu) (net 20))
 (segment (start 147.3838 98.5) (end 148 98.5) (width 0.4064) (layer B.Cu) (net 20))
 (via (at 147.3838 98.5) (size 0.6) (drill 0.4) (layers F.Cu B.Cu) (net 20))
 (segment (start 151.25 96.65) (end 149.5 94.9) (width 0.4064) (layer B.Cu) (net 20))
 (segment (start 151.25 98.5) (end 151.25 96.65) (width 0.4064) (layer B.Cu) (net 20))
 (segment (start 150.5 99.25) (end 151.25 98.5) (width 0.4064) (layer B.Cu) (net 20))
 (segment (start 148.75 99.25) (end 150.5 99.25) (width 0.4064) (layer B.Cu) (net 20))
 (segment (start 148 98.5) (end 148.75 99.25) (width 0.4064) (layer B.Cu) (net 20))
 (segment (start 167.25 94.65) (end 166.9 94.65) (width 0.4064) (layer F.Cu) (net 20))
 (segment (start 147.3838 98.5) (end 146.25 98.5) (width 0.4064) (layer B.Cu) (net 20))
 (segment (start 147.3838 98.5) (end 147.5 98.5) (width 0.3048) (layer B.Cu) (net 20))
 (segment (start 147 96.75) (end 148.65 96.75) (width 0.4064) (layer B.Cu) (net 18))
 (segment (start 148.65 96.75) (end 149.5 97.6) (width 0.4064) (layer B.Cu) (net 18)))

